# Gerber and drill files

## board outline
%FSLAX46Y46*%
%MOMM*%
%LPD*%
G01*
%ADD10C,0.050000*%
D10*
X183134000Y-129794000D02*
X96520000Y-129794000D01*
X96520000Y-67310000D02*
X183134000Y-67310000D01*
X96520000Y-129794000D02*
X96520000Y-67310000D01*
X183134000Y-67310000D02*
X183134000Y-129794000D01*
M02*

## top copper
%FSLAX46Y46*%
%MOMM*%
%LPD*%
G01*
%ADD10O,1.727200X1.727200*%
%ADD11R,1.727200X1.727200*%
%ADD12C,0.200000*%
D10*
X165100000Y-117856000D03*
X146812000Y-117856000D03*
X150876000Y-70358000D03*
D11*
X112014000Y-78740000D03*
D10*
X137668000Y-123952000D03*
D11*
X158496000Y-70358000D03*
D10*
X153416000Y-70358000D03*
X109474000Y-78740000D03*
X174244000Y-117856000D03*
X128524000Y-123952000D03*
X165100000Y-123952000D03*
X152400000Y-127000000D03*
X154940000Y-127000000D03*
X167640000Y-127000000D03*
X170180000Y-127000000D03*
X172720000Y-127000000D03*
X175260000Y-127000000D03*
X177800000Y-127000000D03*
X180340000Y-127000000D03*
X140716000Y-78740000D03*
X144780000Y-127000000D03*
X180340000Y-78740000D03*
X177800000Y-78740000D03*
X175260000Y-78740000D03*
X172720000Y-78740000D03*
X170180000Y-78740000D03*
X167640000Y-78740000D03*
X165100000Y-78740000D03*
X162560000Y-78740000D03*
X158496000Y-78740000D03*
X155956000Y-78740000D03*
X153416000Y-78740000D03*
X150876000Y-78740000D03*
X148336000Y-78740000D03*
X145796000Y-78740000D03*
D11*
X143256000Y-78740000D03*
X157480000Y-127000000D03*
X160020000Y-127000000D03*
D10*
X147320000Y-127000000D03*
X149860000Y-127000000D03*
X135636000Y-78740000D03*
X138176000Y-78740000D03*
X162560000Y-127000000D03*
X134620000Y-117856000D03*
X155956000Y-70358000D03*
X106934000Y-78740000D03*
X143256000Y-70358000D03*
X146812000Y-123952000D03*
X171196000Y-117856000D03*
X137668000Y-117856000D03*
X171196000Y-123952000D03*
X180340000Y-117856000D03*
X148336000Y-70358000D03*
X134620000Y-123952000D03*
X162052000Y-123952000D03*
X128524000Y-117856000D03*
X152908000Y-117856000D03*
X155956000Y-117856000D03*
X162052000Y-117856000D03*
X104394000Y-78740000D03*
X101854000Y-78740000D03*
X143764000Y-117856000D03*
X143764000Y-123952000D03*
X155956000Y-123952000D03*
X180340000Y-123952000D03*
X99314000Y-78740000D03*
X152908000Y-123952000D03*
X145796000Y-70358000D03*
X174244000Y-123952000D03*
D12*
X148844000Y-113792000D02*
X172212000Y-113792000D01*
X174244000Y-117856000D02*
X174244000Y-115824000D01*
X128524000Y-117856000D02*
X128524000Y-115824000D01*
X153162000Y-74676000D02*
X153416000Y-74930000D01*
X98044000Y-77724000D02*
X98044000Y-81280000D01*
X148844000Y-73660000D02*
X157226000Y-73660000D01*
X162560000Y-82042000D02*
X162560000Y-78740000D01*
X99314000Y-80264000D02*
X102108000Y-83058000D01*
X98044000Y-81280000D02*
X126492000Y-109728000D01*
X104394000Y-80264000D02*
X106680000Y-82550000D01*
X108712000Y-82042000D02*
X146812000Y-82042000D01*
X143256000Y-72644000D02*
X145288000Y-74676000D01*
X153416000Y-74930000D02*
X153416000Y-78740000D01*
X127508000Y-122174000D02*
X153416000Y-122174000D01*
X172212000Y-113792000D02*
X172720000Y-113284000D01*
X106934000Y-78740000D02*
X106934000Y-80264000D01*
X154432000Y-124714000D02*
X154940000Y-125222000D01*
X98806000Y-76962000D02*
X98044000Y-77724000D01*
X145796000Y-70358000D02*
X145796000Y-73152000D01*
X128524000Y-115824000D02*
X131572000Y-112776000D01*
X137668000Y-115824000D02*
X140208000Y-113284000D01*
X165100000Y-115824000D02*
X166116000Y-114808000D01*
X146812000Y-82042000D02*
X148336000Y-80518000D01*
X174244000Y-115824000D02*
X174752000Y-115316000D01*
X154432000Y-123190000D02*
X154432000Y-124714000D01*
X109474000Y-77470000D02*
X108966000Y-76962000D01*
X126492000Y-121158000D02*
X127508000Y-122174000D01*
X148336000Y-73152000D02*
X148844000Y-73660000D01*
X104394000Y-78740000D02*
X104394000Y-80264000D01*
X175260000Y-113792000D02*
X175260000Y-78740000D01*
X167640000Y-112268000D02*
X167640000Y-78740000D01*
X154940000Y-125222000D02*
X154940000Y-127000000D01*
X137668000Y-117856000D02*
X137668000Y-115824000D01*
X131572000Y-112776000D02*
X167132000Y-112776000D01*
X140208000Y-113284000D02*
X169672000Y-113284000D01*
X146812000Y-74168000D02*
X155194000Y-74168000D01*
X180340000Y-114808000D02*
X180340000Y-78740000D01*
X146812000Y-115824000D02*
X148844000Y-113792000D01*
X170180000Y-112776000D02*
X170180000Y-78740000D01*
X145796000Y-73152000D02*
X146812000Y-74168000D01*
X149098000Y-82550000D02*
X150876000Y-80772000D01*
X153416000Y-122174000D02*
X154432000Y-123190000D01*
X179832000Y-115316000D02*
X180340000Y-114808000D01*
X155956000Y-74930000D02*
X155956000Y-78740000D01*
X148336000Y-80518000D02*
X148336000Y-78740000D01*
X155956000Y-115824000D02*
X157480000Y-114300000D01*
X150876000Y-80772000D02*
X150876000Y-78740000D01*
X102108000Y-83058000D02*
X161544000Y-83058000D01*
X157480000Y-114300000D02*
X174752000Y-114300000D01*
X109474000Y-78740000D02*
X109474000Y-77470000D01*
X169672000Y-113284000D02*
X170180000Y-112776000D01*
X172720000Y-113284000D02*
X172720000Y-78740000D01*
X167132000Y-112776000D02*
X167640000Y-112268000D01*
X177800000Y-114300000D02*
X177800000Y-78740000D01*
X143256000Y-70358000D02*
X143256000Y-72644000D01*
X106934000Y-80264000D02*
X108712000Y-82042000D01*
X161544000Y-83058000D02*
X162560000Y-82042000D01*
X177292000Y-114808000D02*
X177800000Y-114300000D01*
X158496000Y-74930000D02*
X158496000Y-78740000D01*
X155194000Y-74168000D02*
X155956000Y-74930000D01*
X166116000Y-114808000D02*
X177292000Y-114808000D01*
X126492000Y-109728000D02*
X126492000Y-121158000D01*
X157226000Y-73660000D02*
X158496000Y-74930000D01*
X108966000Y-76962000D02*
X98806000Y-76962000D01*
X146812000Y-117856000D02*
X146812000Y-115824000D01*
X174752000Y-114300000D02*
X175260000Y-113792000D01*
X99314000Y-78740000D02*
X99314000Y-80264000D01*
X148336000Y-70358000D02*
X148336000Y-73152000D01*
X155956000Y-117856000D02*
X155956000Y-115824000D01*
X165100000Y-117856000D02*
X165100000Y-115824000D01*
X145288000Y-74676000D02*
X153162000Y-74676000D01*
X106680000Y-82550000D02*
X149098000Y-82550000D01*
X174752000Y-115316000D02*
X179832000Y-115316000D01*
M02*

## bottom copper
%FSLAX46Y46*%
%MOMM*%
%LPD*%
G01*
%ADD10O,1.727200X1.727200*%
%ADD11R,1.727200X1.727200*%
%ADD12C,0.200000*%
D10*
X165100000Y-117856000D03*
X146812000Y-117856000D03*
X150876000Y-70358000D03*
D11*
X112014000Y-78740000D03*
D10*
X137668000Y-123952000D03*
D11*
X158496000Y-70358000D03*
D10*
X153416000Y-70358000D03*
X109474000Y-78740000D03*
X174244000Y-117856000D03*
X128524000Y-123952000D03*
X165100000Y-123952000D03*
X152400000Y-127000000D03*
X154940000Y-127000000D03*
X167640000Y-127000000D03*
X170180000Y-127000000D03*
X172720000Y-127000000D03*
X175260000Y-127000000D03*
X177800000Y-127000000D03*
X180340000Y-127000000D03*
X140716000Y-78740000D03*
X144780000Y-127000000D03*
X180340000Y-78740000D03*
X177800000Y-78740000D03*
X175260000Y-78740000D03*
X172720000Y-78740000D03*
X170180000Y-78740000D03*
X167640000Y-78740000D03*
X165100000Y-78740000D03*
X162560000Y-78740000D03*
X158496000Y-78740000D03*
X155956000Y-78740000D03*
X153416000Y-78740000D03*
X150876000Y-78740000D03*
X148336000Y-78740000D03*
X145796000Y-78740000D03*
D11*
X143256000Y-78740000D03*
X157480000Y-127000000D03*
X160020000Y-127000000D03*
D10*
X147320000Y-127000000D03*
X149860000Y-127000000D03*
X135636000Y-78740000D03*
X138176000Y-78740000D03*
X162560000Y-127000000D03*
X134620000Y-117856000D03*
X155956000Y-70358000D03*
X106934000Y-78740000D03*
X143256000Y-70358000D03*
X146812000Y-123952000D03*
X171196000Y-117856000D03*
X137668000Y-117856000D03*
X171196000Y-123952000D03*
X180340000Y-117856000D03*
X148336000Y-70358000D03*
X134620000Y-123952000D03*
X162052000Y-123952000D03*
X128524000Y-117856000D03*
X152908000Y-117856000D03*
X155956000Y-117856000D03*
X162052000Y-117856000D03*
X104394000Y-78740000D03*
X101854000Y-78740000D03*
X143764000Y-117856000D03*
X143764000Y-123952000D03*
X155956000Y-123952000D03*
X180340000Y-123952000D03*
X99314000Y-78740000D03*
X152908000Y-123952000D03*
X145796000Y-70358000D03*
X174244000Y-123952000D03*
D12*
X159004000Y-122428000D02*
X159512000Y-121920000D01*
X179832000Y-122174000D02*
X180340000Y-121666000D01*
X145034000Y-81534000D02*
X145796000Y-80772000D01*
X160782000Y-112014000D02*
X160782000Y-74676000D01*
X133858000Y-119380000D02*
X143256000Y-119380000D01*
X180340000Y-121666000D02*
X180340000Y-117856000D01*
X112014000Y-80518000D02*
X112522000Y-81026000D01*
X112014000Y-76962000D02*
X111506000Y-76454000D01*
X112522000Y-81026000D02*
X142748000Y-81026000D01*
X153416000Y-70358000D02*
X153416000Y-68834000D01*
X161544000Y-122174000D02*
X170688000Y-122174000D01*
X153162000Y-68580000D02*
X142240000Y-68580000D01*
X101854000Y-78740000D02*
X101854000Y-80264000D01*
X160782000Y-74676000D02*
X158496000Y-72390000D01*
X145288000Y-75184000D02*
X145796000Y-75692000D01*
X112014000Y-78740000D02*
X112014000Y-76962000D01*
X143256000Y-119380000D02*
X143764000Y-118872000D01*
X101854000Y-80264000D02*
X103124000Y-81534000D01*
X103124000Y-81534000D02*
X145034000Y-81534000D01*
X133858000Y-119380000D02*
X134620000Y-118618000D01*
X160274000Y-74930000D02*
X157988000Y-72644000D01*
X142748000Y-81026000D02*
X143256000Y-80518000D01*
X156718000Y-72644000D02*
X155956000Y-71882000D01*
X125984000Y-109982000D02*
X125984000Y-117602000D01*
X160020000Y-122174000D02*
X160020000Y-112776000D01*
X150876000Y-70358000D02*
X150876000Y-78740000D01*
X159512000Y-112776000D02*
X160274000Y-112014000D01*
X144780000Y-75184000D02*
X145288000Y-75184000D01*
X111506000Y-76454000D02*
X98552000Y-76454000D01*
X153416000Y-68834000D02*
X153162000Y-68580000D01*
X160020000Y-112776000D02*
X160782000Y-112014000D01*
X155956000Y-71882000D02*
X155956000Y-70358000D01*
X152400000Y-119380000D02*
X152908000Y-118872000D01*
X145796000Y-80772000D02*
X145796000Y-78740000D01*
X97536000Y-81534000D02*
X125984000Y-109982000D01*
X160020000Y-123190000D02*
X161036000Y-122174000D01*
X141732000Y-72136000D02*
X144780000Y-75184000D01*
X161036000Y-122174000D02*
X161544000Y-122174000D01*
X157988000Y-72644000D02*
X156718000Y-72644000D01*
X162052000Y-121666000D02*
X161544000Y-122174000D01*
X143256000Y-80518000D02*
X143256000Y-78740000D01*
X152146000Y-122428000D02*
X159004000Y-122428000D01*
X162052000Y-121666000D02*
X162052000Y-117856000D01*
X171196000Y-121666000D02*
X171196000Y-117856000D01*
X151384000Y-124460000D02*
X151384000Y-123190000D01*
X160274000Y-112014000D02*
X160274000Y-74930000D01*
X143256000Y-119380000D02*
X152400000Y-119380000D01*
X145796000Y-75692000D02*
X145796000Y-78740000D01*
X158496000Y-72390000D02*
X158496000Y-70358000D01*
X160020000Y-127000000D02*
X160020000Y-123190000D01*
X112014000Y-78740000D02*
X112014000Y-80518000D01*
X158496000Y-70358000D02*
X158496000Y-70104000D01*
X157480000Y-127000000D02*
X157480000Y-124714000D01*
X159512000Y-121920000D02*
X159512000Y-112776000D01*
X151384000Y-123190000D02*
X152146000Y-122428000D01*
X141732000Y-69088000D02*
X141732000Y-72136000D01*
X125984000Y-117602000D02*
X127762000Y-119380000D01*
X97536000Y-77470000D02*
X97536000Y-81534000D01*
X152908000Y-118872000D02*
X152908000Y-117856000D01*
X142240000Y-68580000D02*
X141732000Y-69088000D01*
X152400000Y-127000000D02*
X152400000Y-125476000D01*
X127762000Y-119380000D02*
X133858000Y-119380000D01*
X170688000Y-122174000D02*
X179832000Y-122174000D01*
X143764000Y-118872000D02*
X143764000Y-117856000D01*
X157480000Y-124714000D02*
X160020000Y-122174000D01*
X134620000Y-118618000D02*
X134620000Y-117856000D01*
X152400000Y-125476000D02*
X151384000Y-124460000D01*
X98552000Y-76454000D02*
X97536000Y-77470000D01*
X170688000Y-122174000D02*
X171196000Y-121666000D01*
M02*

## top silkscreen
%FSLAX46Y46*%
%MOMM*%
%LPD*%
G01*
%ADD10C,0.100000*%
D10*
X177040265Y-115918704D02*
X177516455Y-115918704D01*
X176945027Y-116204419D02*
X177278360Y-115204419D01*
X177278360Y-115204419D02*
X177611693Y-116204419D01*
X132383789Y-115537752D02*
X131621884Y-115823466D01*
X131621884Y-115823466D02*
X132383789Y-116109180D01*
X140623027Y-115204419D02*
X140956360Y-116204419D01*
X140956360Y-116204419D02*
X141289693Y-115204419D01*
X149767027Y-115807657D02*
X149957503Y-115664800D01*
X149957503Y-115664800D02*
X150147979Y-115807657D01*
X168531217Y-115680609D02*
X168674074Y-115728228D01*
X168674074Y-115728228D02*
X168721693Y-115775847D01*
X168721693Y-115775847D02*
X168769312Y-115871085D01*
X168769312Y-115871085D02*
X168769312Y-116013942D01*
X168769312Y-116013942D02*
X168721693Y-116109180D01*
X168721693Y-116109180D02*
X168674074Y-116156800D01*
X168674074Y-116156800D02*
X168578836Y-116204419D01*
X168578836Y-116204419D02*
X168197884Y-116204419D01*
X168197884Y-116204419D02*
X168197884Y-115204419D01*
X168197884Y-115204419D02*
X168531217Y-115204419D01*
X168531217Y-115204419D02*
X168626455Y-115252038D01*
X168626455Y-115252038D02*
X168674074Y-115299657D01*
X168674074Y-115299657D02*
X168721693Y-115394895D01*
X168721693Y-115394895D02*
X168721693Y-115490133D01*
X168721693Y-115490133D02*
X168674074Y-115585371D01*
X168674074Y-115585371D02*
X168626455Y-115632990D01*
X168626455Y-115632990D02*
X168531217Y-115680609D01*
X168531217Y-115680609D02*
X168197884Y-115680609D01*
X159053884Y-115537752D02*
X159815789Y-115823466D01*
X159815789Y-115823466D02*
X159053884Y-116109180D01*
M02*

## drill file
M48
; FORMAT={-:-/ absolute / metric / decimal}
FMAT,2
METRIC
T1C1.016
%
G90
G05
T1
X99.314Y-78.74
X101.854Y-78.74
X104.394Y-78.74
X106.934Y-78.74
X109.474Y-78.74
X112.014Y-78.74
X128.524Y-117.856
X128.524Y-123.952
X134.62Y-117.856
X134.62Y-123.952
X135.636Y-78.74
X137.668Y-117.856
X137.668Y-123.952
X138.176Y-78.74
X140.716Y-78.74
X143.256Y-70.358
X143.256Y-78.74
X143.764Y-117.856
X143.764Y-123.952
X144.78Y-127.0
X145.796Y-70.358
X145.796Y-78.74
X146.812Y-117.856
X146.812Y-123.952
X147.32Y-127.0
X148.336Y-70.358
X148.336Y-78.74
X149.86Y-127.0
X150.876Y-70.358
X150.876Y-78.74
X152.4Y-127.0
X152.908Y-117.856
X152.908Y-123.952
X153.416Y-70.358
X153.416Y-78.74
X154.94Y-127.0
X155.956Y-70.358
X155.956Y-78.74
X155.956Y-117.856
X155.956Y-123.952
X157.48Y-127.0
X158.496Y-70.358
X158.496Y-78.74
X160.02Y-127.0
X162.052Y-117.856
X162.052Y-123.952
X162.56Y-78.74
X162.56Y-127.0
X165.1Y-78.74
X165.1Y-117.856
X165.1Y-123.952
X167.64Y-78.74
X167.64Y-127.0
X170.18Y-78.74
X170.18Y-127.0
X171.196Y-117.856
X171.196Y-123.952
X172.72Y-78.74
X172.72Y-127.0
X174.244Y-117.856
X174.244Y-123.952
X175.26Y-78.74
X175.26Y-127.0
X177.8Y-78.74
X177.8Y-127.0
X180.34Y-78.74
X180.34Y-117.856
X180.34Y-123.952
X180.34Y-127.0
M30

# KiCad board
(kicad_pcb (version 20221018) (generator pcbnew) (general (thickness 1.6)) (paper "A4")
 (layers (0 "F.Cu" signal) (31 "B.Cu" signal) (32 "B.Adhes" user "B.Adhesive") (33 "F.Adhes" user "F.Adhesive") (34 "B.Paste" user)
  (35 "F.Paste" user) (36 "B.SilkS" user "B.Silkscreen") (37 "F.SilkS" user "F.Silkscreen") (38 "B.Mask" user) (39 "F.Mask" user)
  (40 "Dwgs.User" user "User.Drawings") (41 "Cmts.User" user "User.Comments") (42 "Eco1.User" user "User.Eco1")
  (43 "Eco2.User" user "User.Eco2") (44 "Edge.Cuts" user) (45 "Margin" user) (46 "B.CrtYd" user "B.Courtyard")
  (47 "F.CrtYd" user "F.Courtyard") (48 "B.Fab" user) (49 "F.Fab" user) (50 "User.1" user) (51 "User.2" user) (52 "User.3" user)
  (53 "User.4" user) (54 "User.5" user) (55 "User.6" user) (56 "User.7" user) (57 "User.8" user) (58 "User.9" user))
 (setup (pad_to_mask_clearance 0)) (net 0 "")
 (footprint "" (layer "F.Cu") (at 165.1 117.856)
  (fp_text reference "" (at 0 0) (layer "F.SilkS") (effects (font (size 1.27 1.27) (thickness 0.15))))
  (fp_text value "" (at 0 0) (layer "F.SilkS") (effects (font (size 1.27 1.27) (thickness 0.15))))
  (pad "PB5_1" thru_hole oval (at 0 0) (size 1.7272 1.7272) (drill 1.016) (layers "*.Cu" "*.Mask")))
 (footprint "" (layer "F.Cu") (at 146.812 117.856)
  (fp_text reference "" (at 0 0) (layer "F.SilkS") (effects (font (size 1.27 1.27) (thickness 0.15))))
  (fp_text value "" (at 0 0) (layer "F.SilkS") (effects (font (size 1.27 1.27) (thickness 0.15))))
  (pad "PB3_1" thru_hole oval (at 0 0) (size 1.7272 1.7272) (drill 1.016) (layers "*.Cu" "*.Mask")))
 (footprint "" (layer "F.Cu") (at 150.876 70.358)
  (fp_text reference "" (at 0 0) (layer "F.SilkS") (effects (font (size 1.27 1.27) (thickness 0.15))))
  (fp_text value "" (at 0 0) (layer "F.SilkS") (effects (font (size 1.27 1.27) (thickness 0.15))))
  (pad "SDA" thru_hole oval (at 0 0) (size 1.7272 1.7272) (drill 1.016) (layers "*.Cu" "*.Mask")))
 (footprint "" (layer "F.Cu") (at 112.014 78.74)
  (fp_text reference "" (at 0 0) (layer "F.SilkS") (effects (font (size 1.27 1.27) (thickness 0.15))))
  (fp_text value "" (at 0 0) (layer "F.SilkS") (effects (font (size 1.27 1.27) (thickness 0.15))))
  (pad "GND" thru_hole rect (at 0 0) (size 1.7272 1.7272) (drill 1.016) (layers "*.Cu" "*.Mask")))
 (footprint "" (layer "F.Cu") (at 137.668 123.952)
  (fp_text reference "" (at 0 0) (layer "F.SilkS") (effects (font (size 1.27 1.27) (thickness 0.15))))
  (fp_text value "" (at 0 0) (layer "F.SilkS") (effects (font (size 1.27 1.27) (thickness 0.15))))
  (pad "PB2_3" thru_hole oval (at 0 0) (size 1.7272 1.7272) (drill 1.016) (layers "*.Cu" "*.Mask")))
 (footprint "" (layer "F.Cu") (at 158.496 70.358)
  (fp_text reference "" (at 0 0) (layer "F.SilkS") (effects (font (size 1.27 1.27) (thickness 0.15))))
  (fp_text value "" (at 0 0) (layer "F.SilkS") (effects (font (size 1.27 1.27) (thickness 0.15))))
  (pad "GND" thru_hole rect (at 0 0) (size 1.7272 1.7272) (drill 1.016) (layers "*.Cu" "*.Mask")))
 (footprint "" (layer "F.Cu") (at 153.416 70.358)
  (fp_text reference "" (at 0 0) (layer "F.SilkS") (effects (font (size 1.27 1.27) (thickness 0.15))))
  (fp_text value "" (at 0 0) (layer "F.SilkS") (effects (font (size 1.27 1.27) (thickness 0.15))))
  (pad "SCK" thru_hole oval (at 0 0) (size 1.7272 1.7272) (drill 1.016) (layers "*.Cu" "*.Mask")))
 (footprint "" (layer "F.Cu") (at 109.474 78.74)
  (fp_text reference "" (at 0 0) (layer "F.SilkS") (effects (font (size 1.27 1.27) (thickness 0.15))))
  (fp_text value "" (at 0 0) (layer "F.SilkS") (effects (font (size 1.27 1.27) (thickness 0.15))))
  (pad "5V" thru_hole oval (at 0 0) (size 1.7272 1.7272) (drill 1.016) (layers "*.Cu" "*.Mask")))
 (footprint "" (layer "F.Cu") (at 174.244 117.856)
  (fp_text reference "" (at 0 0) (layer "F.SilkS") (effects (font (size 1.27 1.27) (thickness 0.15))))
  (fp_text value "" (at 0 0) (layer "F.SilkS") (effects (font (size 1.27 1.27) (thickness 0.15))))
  (pad "PB6_1" thru_hole oval (at 0 0) (size 1.7272 1.7272) (drill 1.016) (layers "*.Cu" "*.Mask")))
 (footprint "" (layer "F.Cu") (at 128.524 123.952)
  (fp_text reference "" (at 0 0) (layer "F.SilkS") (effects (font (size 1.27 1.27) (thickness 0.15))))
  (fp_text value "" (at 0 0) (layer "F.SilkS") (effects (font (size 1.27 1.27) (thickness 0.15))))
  (pad "PB1_3" thru_hole oval (at 0 0) (size 1.7272 1.7272) (drill 1.016) (layers "*.Cu" "*.Mask")))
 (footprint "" (layer "F.Cu") (at 165.1 123.952)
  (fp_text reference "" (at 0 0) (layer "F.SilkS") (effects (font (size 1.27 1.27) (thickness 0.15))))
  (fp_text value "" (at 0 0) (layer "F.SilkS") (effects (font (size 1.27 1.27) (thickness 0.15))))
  (pad "PB5_3" thru_hole oval (at 0 0) (size 1.7272 1.7272) (drill 1.016) (layers "*.Cu" "*.Mask")))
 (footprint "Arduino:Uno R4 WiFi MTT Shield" (layer "F.Cu") (at 116.84 129.54)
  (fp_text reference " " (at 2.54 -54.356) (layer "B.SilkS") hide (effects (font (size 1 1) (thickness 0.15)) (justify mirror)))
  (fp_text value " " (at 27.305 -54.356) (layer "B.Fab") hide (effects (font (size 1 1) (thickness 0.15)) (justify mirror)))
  (pad "3V3" thru_hole oval (at 35.56 -2.54) (size 1.7272 1.7272) (drill 1.016) (layers "*.Cu" "*.Mask"))
  (pad "5V1" thru_hole oval (at 38.1 -2.54) (size 1.7272 1.7272) (drill 1.016) (layers "*.Cu" "*.Mask"))
  (pad "A0" thru_hole oval (at 50.8 -2.54) (size 1.7272 1.7272) (drill 1.016) (layers "*.Cu" "*.Mask"))
  (pad "A1" thru_hole oval (at 53.34 -2.54) (size 1.7272 1.7272) (drill 1.016) (layers "*.Cu" "*.Mask"))
  (pad "A2" thru_hole oval (at 55.88 -2.54) (size 1.7272 1.7272) (drill 1.016) (layers "*.Cu" "*.Mask"))
  (pad "A3" thru_hole oval (at 58.42 -2.54) (size 1.7272 1.7272) (drill 1.016) (layers "*.Cu" "*.Mask"))
  (pad "A4" thru_hole oval (at 60.96 -2.54) (size 1.7272 1.7272) (drill 1.016) (layers "*.Cu" "*.Mask"))
  (pad "A5" thru_hole oval (at 63.5 -2.54) (size 1.7272 1.7272) (drill 1.016) (layers "*.Cu" "*.Mask"))
  (pad "AREF" thru_hole oval (at 23.876 -50.8) (size 1.7272 1.7272) (drill 1.016) (layers "*.Cu" "*.Mask"))
  (pad "BOOT" thru_hole oval (at 27.94 -2.54) (size 1.7272 1.7272) (drill 1.016) (layers "*.Cu" "*.Mask"))
  (pad "D0" thru_hole oval (at 63.5 -50.8) (size 1.7272 1.7272) (drill 1.016) (layers "*.Cu" "*.Mask"))
  (pad "D1" thru_hole oval (at 60.96 -50.8) (size 1.7272 1.7272) (drill 1.016) (layers "*.Cu" "*.Mask"))
  (pad "D2" thru_hole oval (at 58.42 -50.8) (size 1.7272 1.7272) (drill 1.016) (layers "*.Cu" "*.Mask"))
  (pad "D3" thru_hole oval (at 55.88 -50.8) (size 1.7272 1.7272) (drill 1.016) (layers "*.Cu" "*.Mask"))
  (pad "D4" thru_hole oval (at 53.34 -50.8) (size 1.7272 1.7272) (drill 1.016) (layers "*.Cu" "*.Mask"))
  (pad "D5" thru_hole oval (at 50.8 -50.8) (size 1.7272 1.7272) (drill 1.016) (layers "*.Cu" "*.Mask"))
  (pad "D6" thru_hole oval (at 48.26 -50.8) (size 1.7272 1.7272) (drill 1.016) (layers "*.Cu" "*.Mask"))
  (pad "D7" thru_hole oval (at 45.72 -50.8) (size 1.7272 1.7272) (drill 1.016) (layers "*.Cu" "*.Mask"))
  (pad "D8" thru_hole oval (at 41.656 -50.8) (size 1.7272 1.7272) (drill 1.016) (layers "*.Cu" "*.Mask"))
  (pad "D9" thru_hole oval (at 39.116 -50.8) (size 1.7272 1.7272) (drill 1.016) (layers "*.Cu" "*.Mask"))
  (pad "D10" thru_hole oval (at 36.576 -50.8) (size 1.7272 1.7272) (drill 1.016) (layers "*.Cu" "*.Mask"))
  (pad "D11" thru_hole oval (at 34.036 -50.8) (size 1.7272 1.7272) (drill 1.016) (layers "*.Cu" "*.Mask"))
  (pad "D12" thru_hole oval (at 31.496 -50.8) (size 1.7272 1.7272) (drill 1.016) (layers "*.Cu" "*.Mask"))
  (pad "D13" thru_hole oval (at 28.956 -50.8) (size 1.7272 1.7272) (drill 1.016) (layers "*.Cu" "*.Mask"))
  (pad "GND1" thru_hole rect (at 26.416 -50.8) (size 1.7272 1.7272) (drill 1.016) (layers "*.Cu" "*.Mask"))
  (pad "GND2" thru_hole rect (at 40.64 -2.54) (size 1.7272 1.7272) (drill 1.016) (layers "*.Cu" "*.Mask"))
  (pad "GND3" thru_hole rect (at 43.18 -2.54) (size 1.7272 1.7272) (drill 1.016) (layers "*.Cu" "*.Mask"))
  (pad "IORF" thru_hole oval (at 30.48 -2.54) (size 1.7272 1.7272) (drill 1.016) (layers "*.Cu" "*.Mask"))
  (pad "RST1" thru_hole oval (at 33.02 -2.54) (size 1.7272 1.7272) (drill 1.016) (layers "*.Cu" "*.Mask"))
  (pad "SCL" thru_hole oval (at 18.796 -50.8) (size 1.7272 1.7272) (drill 1.016) (layers "*.Cu" "*.Mask"))
  (pad "SDA" thru_hole oval (at 21.336 -50.8) (size 1.7272 1.7272) (drill 1.016) (layers "*.Cu" "*.Mask"))
  (pad "VIN" thru_hole oval (at 45.72 -2.54) (size 1.7272 1.7272) (drill 1.016) (layers "*.Cu" "*.Mask")))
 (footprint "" (layer "F.Cu") (at 134.62 117.856)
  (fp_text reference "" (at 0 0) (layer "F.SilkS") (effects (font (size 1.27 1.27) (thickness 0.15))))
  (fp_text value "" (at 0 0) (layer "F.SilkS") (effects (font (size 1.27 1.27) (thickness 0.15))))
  (pad "PB1_2" thru_hole oval (at 0 0) (size 1.7272 1.7272) (drill 1.016) (layers "*.Cu" "*.Mask")))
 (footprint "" (layer "F.Cu") (at 155.956 70.358)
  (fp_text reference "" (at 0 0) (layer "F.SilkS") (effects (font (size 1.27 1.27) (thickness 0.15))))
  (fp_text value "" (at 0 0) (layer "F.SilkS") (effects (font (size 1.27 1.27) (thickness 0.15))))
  (pad "3V3" thru_hole oval (at 0 0) (size 1.7272 1.7272) (drill 1.016) (layers "*.Cu" "*.Mask")))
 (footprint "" (layer "F.Cu") (at 106.934 78.74)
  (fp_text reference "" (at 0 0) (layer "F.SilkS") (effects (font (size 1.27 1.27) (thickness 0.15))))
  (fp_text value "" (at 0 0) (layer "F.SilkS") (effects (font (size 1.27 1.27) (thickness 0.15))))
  (pad "MISO" thru_hole oval (at 0 0) (size 1.7272 1.7272) (drill 1.016) (layers "*.Cu" "*.Mask")))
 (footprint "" (layer "F.Cu") (at 143.256 70.358)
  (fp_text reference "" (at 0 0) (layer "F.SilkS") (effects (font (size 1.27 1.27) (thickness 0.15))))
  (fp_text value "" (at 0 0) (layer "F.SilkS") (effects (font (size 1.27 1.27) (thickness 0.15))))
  (pad "CS" thru_hole oval (at 0 0) (size 1.7272 1.7272) (drill 1.016) (layers "*.Cu" "*.Mask")))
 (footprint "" (layer "F.Cu") (at 146.812 123.952)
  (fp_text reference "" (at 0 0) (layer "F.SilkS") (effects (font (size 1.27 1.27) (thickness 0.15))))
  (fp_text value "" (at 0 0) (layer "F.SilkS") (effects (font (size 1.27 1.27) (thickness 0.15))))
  (pad "PB3_3" thru_hole oval (at 0 0) (size 1.7272 1.7272) (drill 1.016) (layers "*.Cu" "*.Mask")))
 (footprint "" (layer "F.Cu") (at 171.196 117.856)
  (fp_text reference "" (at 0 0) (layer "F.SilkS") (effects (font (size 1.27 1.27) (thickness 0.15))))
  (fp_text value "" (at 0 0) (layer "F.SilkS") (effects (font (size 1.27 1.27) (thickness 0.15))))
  (pad "PB5_2" thru_hole oval (at 0 0) (size 1.7272 1.7272) (drill 1.016) (layers "*.Cu" "*.Mask")))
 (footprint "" (layer "F.Cu") (at 137.668 117.856)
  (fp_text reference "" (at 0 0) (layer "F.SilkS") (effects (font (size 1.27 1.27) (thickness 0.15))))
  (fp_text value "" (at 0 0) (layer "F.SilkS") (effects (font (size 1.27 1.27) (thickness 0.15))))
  (pad "PB2_1" thru_hole oval (at 0 0) (size 1.7272 1.7272) (drill 1.016) (layers "*.Cu" "*.Mask")))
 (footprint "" (layer "F.Cu") (at 171.196 123.952)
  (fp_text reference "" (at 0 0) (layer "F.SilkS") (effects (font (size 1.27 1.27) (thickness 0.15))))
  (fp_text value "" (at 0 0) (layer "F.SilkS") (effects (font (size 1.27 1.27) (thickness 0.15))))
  (pad "PB5_4" thru_hole oval (at 0 0) (size 1.7272 1.7272) (drill 1.016) (layers "*.Cu" "*.Mask")))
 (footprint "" (layer "F.Cu") (at 180.34 117.856)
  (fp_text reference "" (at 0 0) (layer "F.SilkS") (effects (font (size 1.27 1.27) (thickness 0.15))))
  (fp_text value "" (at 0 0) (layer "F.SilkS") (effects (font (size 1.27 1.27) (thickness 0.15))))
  (pad "PB6_2" thru_hole oval (at 0 0) (size 1.7272 1.7272) (drill 1.016) (layers "*.Cu" "*.Mask")))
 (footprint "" (layer "F.Cu") (at 148.336 70.358)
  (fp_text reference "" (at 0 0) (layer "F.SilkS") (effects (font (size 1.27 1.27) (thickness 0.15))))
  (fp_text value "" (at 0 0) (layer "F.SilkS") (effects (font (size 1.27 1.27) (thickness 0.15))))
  (pad "RES" thru_hole oval (at 0 0) (size 1.7272 1.7272) (drill 1.016) (layers "*.Cu" "*.Mask")))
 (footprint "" (layer "F.Cu") (at 134.62 123.952)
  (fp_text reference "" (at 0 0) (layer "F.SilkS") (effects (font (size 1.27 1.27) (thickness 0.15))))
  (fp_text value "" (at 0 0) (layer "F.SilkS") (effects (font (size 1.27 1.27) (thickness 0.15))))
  (pad "PB1_4" thru_hole oval (at 0 0) (size 1.7272 1.7272) (drill 1.016) (layers "*.Cu" "*.Mask")))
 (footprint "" (layer "F.Cu") (at 162.052 123.952)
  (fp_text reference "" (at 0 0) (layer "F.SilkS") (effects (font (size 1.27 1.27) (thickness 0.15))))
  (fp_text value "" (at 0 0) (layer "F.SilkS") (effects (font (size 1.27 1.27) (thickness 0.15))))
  (pad "PB4_4" thru_hole oval (at 0 0) (size 1.7272 1.7272) (drill 1.016) (layers "*.Cu" "*.Mask")))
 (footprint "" (layer "F.Cu") (at 128.524 117.856)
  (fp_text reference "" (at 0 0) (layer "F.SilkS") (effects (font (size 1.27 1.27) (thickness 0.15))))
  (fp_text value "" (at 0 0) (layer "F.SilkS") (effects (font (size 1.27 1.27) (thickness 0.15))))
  (pad "PB1_1" thru_hole oval (at 0 0) (size 1.7272 1.7272) (drill 1.016) (layers "*.Cu" "*.Mask")))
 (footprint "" (layer "F.Cu") (at 152.908 117.856)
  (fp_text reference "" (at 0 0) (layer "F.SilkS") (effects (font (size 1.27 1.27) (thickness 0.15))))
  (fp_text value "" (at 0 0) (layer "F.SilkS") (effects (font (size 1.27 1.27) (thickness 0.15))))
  (pad "PB3_2" thru_hole oval (at 0 0) (size 1.7272 1.7272) (drill 1.016) (layers "*.Cu" "*.Mask")))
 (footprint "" (layer "F.Cu") (at 155.956 117.856)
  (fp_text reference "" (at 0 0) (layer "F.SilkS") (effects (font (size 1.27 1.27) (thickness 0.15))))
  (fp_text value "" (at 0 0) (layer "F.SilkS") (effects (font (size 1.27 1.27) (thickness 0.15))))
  (pad "PB4_1" thru_hole oval (at 0 0) (size 1.7272 1.7272) (drill 1.016) (layers "*.Cu" "*.Mask")))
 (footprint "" (layer "F.Cu") (at 162.052 117.856)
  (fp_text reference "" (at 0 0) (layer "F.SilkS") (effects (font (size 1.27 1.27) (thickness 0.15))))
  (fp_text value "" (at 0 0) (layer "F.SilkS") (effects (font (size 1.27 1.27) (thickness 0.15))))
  (pad "PB4_2" thru_hole oval (at 0 0) (size 1.7272 1.7272) (drill 1.016) (layers "*.Cu" "*.Mask")))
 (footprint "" (layer "F.Cu") (at 104.394 78.74)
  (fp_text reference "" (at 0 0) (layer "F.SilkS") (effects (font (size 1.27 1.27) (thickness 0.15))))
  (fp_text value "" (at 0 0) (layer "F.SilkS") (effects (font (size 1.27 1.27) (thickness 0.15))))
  (pad "MOSI" thru_hole oval (at 0 0) (size 1.7272 1.7272) (drill 1.016) (layers "*.Cu" "*.Mask")))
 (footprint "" (layer "F.Cu") (at 101.854 78.74)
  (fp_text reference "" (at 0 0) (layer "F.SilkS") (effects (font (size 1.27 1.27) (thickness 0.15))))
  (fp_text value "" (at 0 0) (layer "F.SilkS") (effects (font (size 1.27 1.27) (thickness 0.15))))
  (pad "SCK" thru_hole oval (at 0 0) (size 1.7272 1.7272) (drill 1.016) (layers "*.Cu" "*.Mask")))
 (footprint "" (layer "F.Cu") (at 143.764 117.856)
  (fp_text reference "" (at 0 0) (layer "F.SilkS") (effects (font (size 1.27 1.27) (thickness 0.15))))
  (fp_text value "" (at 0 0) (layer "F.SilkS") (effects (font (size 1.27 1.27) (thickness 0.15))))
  (pad "PB2_2" thru_hole oval (at 0 0) (size 1.7272 1.7272) (drill 1.016) (layers "*.Cu" "*.Mask")))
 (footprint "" (layer "F.Cu") (at 143.764 123.952)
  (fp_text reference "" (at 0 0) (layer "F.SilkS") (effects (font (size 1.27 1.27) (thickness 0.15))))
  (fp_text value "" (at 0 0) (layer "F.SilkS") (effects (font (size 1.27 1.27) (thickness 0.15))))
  (pad "PB2_4" thru_hole oval (at 0 0) (size 1.7272 1.7272) (drill 1.016) (layers "*.Cu" "*.Mask")))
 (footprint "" (layer "F.Cu") (at 155.956 123.952)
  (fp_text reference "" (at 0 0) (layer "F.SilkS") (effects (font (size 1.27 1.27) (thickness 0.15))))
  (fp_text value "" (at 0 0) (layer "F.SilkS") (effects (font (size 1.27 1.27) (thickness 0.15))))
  (pad "PB4_3" thru_hole oval (at 0 0) (size 1.7272 1.7272) (drill 1.016) (layers "*.Cu" "*.Mask")))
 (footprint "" (layer "F.Cu") (at 180.34 123.952)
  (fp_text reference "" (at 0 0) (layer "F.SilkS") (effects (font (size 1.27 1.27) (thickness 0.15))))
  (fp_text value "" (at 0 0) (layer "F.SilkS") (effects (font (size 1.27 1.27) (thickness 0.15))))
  (pad "PB6_4" thru_hole oval (at 0 0) (size 1.7272 1.7272) (drill 1.016) (layers "*.Cu" "*.Mask")))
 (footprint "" (layer "F.Cu") (at 99.314 78.74)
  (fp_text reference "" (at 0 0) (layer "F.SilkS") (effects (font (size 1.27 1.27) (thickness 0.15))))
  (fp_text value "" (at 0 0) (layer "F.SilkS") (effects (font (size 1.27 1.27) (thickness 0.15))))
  (pad "CS" thru_hole oval (at 0 0) (size 1.7272 1.7272) (drill 1.016) (layers "*.Cu" "*.Mask")))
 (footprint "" (layer "F.Cu") (at 152.908 123.952)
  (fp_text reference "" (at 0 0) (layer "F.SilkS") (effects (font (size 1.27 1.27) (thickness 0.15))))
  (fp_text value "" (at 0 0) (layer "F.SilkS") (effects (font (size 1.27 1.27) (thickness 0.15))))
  (pad "PB3_4" thru_hole oval (at 0 0) (size 1.7272 1.7272) (drill 1.016) (layers "*.Cu" "*.Mask")))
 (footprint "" (layer "F.Cu") (at 145.796 70.358)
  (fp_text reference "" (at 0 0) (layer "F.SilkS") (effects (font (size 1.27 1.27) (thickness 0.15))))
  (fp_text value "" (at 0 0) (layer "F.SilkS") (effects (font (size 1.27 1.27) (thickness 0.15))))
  (pad "DC" thru_hole oval (at 0 0) (size 1.7272 1.7272) (drill 1.016) (layers "*.Cu" "*.Mask")))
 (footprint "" (layer "F.Cu") (at 174.244 123.952)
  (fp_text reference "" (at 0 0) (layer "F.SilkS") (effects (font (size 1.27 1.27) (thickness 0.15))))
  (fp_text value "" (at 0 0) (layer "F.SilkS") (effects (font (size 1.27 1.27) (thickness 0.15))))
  (pad "PB6_3" thru_hole oval (at 0 0) (size 1.7272 1.7272) (drill 1.016) (layers "*.Cu" "*.Mask")))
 (gr_line (start 183.134 129.794) (end 96.52 129.794) (stroke (width 0.05) (type default)) (layer "Edge.Cuts"))
 (gr_line (start 96.52 67.31) (end 183.134 67.31) (stroke (width 0.05) (type default)) (layer "Edge.Cuts"))
 (gr_line (start 96.52 129.794) (end 96.52 67.31) (stroke (width 0.05) (type default)) (layer "Edge.Cuts"))
 (gr_line (start 183.134 67.31) (end 183.134 129.794) (stroke (width 0.05) (type default)) (layer "Edge.Cuts"))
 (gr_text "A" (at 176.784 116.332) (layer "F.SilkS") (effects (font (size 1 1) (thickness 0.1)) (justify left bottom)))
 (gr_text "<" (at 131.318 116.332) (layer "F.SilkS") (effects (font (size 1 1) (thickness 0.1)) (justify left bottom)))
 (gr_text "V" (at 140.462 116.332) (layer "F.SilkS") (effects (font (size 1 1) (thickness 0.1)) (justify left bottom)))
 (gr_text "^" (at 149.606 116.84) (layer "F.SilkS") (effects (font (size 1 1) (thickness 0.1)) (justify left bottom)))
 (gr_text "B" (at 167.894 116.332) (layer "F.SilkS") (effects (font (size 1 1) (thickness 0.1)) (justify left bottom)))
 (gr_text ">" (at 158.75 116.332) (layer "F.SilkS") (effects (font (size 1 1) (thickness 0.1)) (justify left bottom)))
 (segment (start 148.844 113.792) (end 172.212 113.792) (width 0.2) (layer "F.Cu") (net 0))
 (segment (start 174.244 117.856) (end 174.244 115.824) (width 0.2) (layer "F.Cu") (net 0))
 (segment (start 128.524 117.856) (end 128.524 115.824) (width 0.2) (layer "F.Cu") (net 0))
 (segment (start 153.162 74.676) (end 153.416 74.93) (width 0.2) (layer "F.Cu") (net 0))
 (segment (start 98.044 77.724) (end 98.044 81.28) (width 0.2) (layer "F.Cu") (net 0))
 (segment (start 148.844 73.66) (end 157.226 73.66) (width 0.2) (layer "F.Cu") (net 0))
 (segment (start 162.56 82.042) (end 162.56 78.74) (width 0.2) (layer "F.Cu") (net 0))
 (segment (start 99.314 80.264) (end 102.108 83.058) (width 0.2) (layer "F.Cu") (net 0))
 (segment (start 98.044 81.28) (end 126.492 109.728) (width 0.2) (layer "F.Cu") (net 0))
 (segment (start 104.394 80.264) (end 106.68 82.55) (width 0.2) (layer "F.Cu") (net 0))
 (segment (start 108.712 82.042) (end 146.812 82.042) (width 0.2) (layer "F.Cu") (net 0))
 (segment (start 143.256 72.644) (end 145.288 74.676) (width 0.2) (layer "F.Cu") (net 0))
 (segment (start 153.416 74.93) (end 153.416 78.74) (width 0.2) (layer "F.Cu") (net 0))
 (segment (start 127.508 122.174) (end 153.416 122.174) (width 0.2) (layer "F.Cu") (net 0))
 (segment (start 172.212 113.792) (end 172.72 113.284) (width 0.2) (layer "F.Cu") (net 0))
 (segment (start 106.934 78.74) (end 106.934 80.264) (width 0.2) (layer "F.Cu") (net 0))
 (segment (start 154.432 124.714) (end 154.94 125.222) (width 0.2) (layer "F.Cu") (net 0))
 (segment (start 98.806 76.962) (end 98.044 77.724) (width 0.2) (layer "F.Cu") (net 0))
 (segment (start 145.796 70.358) (end 145.796 73.152) (width 0.2) (layer "F.Cu") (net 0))
 (segment (start 128.524 115.824) (end 131.572 112.776) (width 0.2) (layer "F.Cu") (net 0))
 (segment (start 137.668 115.824) (end 140.208 113.284) (width 0.2) (layer "F.Cu") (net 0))
 (segment (start 165.1 115.824) (end 166.116 114.808) (width 0.2) (layer "F.Cu") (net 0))
 (segment (start 146.812 82.042) (end 148.336 80.518) (width 0.2) (layer "F.Cu") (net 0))
 (segment (start 174.244 115.824) (end 174.752 115.316) (width 0.2) (layer "F.Cu") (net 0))
 (segment (start 154.432 123.19) (end 154.432 124.714) (width 0.2) (layer "F.Cu") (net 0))
 (segment (start 109.474 77.47) (end 108.966 76.962) (width 0.2) (layer "F.Cu") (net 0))
 (segment (start 126.492 121.158) (end 127.508 122.174) (width 0.2) (layer "F.Cu") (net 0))
 (segment (start 148.336 73.152) (end 148.844 73.66) (width 0.2) (layer "F.Cu") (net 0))
 (segment (start 104.394 78.74) (end 104.394 80.264) (width 0.2) (layer "F.Cu") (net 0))
 (segment (start 175.26 113.792) (end 175.26 78.74) (width 0.2) (layer "F.Cu") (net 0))
 (segment (start 167.64 112.268) (end 167.64 78.74) (width 0.2) (layer "F.Cu") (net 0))
 (segment (start 154.94 125.222) (end 154.94 127) (width 0.2) (layer "F.Cu") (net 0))
 (segment (start 137.668 117.856) (end 137.668 115.824) (width 0.2) (layer "F.Cu") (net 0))
 (segment (start 131.572 112.776) (end 167.132 112.776) (width 0.2) (layer "F.Cu") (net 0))
 (segment (start 140.208 113.284) (end 169.672 113.284) (width 0.2) (layer "F.Cu") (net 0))
 (segment (start 146.812 74.168) (end 155.194 74.168) (width 0.2) (layer "F.Cu") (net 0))
 (segment (start 180.34 114.808) (end 180.34 78.74) (width 0.2) (layer "F.Cu") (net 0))
 (segment (start 146.812 115.824) (end 148.844 113.792) (width 0.2) (layer "F.Cu") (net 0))
 (segment (start 170.18 112.776) (end 170.18 78.74) (width 0.2) (layer "F.Cu") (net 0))
 (segment (start 145.796 73.152) (end 146.812 74.168) (width 0.2) (layer "F.Cu") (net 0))
 (segment (start 149.098 82.55) (end 150.876 80.772) (width 0.2) (layer "F.Cu") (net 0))
 (segment (start 153.416 122.174) (end 154.432 123.19) (width 0.2) (layer "F.Cu") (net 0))
 (segment (start 179.832 115.316) (end 180.34 114.808) (width 0.2) (layer "F.Cu") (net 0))
 (segment (start 155.956 74.93) (end 155.956 78.74) (width 0.2) (layer "F.Cu") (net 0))
 (segment (start 148.336 80.518) (end 148.336 78.74) (width 0.2) (layer "F.Cu") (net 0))
 (segment (start 155.956 115.824) (end 157.48 114.3) (width 0.2) (layer "F.Cu") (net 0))
 (segment (start 150.876 80.772) (end 150.876 78.74) (width 0.2) (layer "F.Cu") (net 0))
 (segment (start 102.108 83.058) (end 161.544 83.058) (width 0.2) (layer "F.Cu") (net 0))
 (segment (start 157.48 114.3) (end 174.752 114.3) (width 0.2) (layer "F.Cu") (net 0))
 (segment (start 109.474 78.74) (end 109.474 77.47) (width 0.2) (layer "F.Cu") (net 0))
 (segment (start 169.672 113.284) (end 170.18 112.776) (width 0.2) (layer "F.Cu") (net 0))
 (segment (start 172.72 113.284) (end 172.72 78.74) (width 0.2) (layer "F.Cu") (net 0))
 (segment (start 167.132 112.776) (end 167.64 112.268) (width 0.2) (layer "F.Cu") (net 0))
 (segment (start 177.8 114.3) (end 177.8 78.74) (width 0.2) (layer "F.Cu") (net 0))
 (segment (start 143.256 70.358) (end 143.256 72.644) (width 0.2) (layer "F.Cu") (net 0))
 (segment (start 106.934 80.264) (end 108.712 82.042) (width 0.2) (layer "F.Cu") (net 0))
 (segment (start 161.544 83.058) (end 162.56 82.042) (width 0.2) (layer "F.Cu") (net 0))
 (segment (start 177.292 114.808) (end 177.8 114.3) (width 0.2) (layer "F.Cu") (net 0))
 (segment (start 158.496 74.93) (end 158.496 78.74) (width 0.2) (layer "F.Cu") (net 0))
 (segment (start 155.194 74.168) (end 155.956 74.93) (width 0.2) (layer "F.Cu") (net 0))
 (segment (start 166.116 114.808) (end 177.292 114.808) (width 0.2) (layer "F.Cu") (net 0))
 (segment (start 126.492 109.728) (end 126.492 121.158) (width 0.2) (layer "F.Cu") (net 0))
 (segment (start 157.226 73.66) (end 158.496 74.93) (width 0.2) (layer "F.Cu") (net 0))
 (segment (start 108.966 76.962) (end 98.806 76.962) (width 0.2) (layer "F.Cu") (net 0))
 (segment (start 146.812 117.856) (end 146.812 115.824) (width 0.2) (layer "F.Cu") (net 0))
 (segment (start 174.752 114.3) (end 175.26 113.792) (width 0.2) (layer "F.Cu") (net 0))
 (segment (start 99.314 78.74) (end 99.314 80.264) (width 0.2) (layer "F.Cu") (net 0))
 (segment (start 148.336 70.358) (end 148.336 73.152) (width 0.2) (layer "F.Cu") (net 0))
 (segment (start 155.956 117.856) (end 155.956 115.824) (width 0.2) (layer "F.Cu") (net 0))
 (segment (start 165.1 117.856) (end 165.1 115.824) (width 0.2) (layer "F.Cu") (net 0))
 (segment (start 145.288 74.676) (end 153.162 74.676) (width 0.2) (layer "F.Cu") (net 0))
 (segment (start 106.68 82.55) (end 149.098 82.55) (width 0.2) (layer "F.Cu") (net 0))
 (segment (start 174.752 115.316) (end 179.832 115.316) (width 0.2) (layer "F.Cu") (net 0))
 (segment (start 159.004 122.428) (end 159.512 121.92) (width 0.2) (layer "B.Cu") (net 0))
 (segment (start 179.832 122.174) (end 180.34 121.666) (width 0.2) (layer "B.Cu") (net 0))
 (segment (start 145.034 81.534) (end 145.796 80.772) (width 0.2) (layer "B.Cu") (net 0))
 (segment (start 160.782 112.014) (end 160.782 74.676) (width 0.2) (layer "B.Cu") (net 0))
 (segment (start 133.858 119.38) (end 143.256 119.38) (width 0.2) (layer "B.Cu") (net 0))
 (segment (start 180.34 121.666) (end 180.34 117.856) (width 0.2) (layer "B.Cu") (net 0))
 (segment (start 112.014 80.518) (end 112.522 81.026) (width 0.2) (layer "B.Cu") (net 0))
 (segment (start 112.014 76.962) (end 111.506 76.454) (width 0.2) (layer "B.Cu") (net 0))
 (segment (start 112.522 81.026) (end 142.748 81.026) (width 0.2) (layer "B.Cu") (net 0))
 (segment (start 153.416 70.358) (end 153.416 68.834) (width 0.2) (layer "B.Cu") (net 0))
 (segment (start 161.544 122.174) (end 170.688 122.174) (width 0.2) (layer "B.Cu") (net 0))
 (segment (start 153.162 68.58) (end 142.24 68.58) (width 0.2) (layer "B.Cu") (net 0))
 (segment (start 101.854 78.74) (end 101.854 80.264) (width 0.2) (layer "B.Cu") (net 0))
 (segment (start 160.782 74.676) (end 158.496 72.39) (width 0.2) (layer "B.Cu") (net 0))
 (segment (start 145.288 75.184) (end 145.796 75.692) (width 0.2) (layer "B.Cu") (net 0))
 (segment (start 112.014 78.74) (end 112.014 76.962) (width 0.2) (layer "B.Cu") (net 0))
 (segment (start 143.256 119.38) (end 143.764 118.872) (width 0.2) (layer "B.Cu") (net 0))
 (segment (start 101.854 80.264) (end 103.124 81.534) (width 0.2) (layer "B.Cu") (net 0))
 (segment (start 103.124 81.534) (end 145.034 81.534) (width 0.2) (layer "B.Cu") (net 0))
 (segment (start 133.858 119.38) (end 134.62 118.618) (width 0.2) (layer "B.Cu") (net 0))
 (segment (start 160.274 74.93) (end 157.988 72.644) (width 0.2) (layer "B.Cu") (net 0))
 (segment (start 142.748 81.026) (end 143.256 80.518) (width 0.2) (layer "B.Cu") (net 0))
 (segment (start 156.718 72.644) (end 155.956 71.882) (width 0.2) (layer "B.Cu") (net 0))
 (segment (start 125.984 109.982) (end 125.984 117.602) (width 0.2) (layer "B.Cu") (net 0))
 (segment (start 160.02 122.174) (end 160.02 112.776) (width 0.2) (layer "B.Cu") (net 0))
 (segment (start 150.876 70.358) (end 150.876 78.74) (width 0.2) (layer "B.Cu") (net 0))
 (segment (start 159.512 112.776) (end 160.274 112.014) (width 0.2) (layer "B.Cu") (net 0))
 (segment (start 144.78 75.184) (end 145.288 75.184) (width 0.2) (layer "B.Cu") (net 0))
 (segment (start 111.506 76.454) (end 98.552 76.454) (width 0.2) (layer "B.Cu") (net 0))
 (segment (start 153.416 68.834) (end 153.162 68.58) (width 0.2) (layer "B.Cu") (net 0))
 (segment (start 160.02 112.776) (end 160.782 112.014) (width 0.2) (layer "B.Cu") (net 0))
 (segment (start 155.956 71.882) (end 155.956 70.358) (width 0.2) (layer "B.Cu") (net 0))
 (segment (start 152.4 119.38) (end 152.908 118.872) (width 0.2) (layer "B.Cu") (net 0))
 (segment (start 145.796 80.772) (end 145.796 78.74) (width 0.2) (layer "B.Cu") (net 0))
 (segment (start 97.536 81.534) (end 125.984 109.982) (width 0.2) (layer "B.Cu") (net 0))
 (segment (start 160.02 123.19) (end 161.036 122.174) (width 0.2) (layer "B.Cu") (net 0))
 (segment (start 141.732 72.136) (end 144.78 75.184) (width 0.2) (layer "B.Cu") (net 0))
 (segment (start 161.036 122.174) (end 161.544 122.174) (width 0.2) (layer "B.Cu") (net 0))
 (segment (start 157.988 72.644) (end 156.718 72.644) (width 0.2) (layer "B.Cu") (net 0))
 (segment (start 162.052 121.666) (end 161.544 122.174) (width 0.2) (layer "B.Cu") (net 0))
 (segment (start 143.256 80.518) (end 143.256 78.74) (width 0.2) (layer "B.Cu") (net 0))
 (segment (start 152.146 122.428) (end 159.004 122.428) (width 0.2) (layer "B.Cu") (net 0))
 (segment (start 162.052 121.666) (end 162.052 117.856) (width 0.2) (layer "B.Cu") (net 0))
 (segment (start 171.196 121.666) (end 171.196 117.856) (width 0.2) (layer "B.Cu") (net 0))
 (segment (start 151.384 124.46) (end 151.384 123.19) (width 0.2) (layer "B.Cu") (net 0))
 (segment (start 160.274 112.014) (end 160.274 74.93) (width 0.2) (layer "B.Cu") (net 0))
 (segment (start 143.256 119.38) (end 152.4 119.38) (width 0.2) (layer "B.Cu") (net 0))
 (segment (start 145.796 75.692) (end 145.796 78.74) (width 0.2) (layer "B.Cu") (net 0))
 (segment (start 158.496 72.39) (end 158.496 70.358) (width 0.2) (layer "B.Cu") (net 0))
 (segment (start 160.02 127) (end 160.02 123.19) (width 0.2) (layer "B.Cu") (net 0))
 (segment (start 112.014 78.74) (end 112.014 80.518) (width 0.2) (layer "B.Cu") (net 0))
 (segment (start 158.496 70.358) (end 158.496 70.104) (width 0.2) (layer "B.Cu") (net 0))
 (segment (start 157.48 127) (end 157.48 124.714) (width 0.2) (layer "B.Cu") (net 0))
 (segment (start 159.512 121.92) (end 159.512 112.776) (width 0.2) (layer "B.Cu") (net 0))
 (segment (start 151.384 123.19) (end 152.146 122.428) (width 0.2) (layer "B.Cu") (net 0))
 (segment (start 141.732 69.088) (end 141.732 72.136) (width 0.2) (layer "B.Cu") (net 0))
 (segment (start 125.984 117.602) (end 127.762 119.38) (width 0.2) (layer "B.Cu") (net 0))
 (segment (start 97.536 77.47) (end 97.536 81.534) (width 0.2) (layer "B.Cu") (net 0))
 (segment (start 152.908 118.872) (end 152.908 117.856) (width 0.2) (layer "B.Cu") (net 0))
 (segment (start 142.24 68.58) (end 141.732 69.088) (width 0.2) (layer "B.Cu") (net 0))
 (segment (start 152.4 127) (end 152.4 125.476) (width 0.2) (layer "B.Cu") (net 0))
 (segment (start 127.762 119.38) (end 133.858 119.38) (width 0.2) (layer "B.Cu") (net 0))
 (segment (start 170.688 122.174) (end 179.832 122.174) (width 0.2) (layer "B.Cu") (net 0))
 (segment (start 143.764 118.872) (end 143.764 117.856) (width 0.2) (layer "B.Cu") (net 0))
 (segment (start 157.48 124.714) (end 160.02 122.174) (width 0.2) (layer "B.Cu") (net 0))
 (segment (start 134.62 118.618) (end 134.62 117.856) (width 0.2) (layer "B.Cu") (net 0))
 (segment (start 152.4 125.476) (end 151.384 124.46) (width 0.2) (layer "B.Cu") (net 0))
 (segment (start 98.552 76.454) (end 97.536 77.47) (width 0.2) (layer "B.Cu") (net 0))
 (segment (start 170.688 122.174) (end 171.196 121.666) (width 0.2) (layer "B.Cu") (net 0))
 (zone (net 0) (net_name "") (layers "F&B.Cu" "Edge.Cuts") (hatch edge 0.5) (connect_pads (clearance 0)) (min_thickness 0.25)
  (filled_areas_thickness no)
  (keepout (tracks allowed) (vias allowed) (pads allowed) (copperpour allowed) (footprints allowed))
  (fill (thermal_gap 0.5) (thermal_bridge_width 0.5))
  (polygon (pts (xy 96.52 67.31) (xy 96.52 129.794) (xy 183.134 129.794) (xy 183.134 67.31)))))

